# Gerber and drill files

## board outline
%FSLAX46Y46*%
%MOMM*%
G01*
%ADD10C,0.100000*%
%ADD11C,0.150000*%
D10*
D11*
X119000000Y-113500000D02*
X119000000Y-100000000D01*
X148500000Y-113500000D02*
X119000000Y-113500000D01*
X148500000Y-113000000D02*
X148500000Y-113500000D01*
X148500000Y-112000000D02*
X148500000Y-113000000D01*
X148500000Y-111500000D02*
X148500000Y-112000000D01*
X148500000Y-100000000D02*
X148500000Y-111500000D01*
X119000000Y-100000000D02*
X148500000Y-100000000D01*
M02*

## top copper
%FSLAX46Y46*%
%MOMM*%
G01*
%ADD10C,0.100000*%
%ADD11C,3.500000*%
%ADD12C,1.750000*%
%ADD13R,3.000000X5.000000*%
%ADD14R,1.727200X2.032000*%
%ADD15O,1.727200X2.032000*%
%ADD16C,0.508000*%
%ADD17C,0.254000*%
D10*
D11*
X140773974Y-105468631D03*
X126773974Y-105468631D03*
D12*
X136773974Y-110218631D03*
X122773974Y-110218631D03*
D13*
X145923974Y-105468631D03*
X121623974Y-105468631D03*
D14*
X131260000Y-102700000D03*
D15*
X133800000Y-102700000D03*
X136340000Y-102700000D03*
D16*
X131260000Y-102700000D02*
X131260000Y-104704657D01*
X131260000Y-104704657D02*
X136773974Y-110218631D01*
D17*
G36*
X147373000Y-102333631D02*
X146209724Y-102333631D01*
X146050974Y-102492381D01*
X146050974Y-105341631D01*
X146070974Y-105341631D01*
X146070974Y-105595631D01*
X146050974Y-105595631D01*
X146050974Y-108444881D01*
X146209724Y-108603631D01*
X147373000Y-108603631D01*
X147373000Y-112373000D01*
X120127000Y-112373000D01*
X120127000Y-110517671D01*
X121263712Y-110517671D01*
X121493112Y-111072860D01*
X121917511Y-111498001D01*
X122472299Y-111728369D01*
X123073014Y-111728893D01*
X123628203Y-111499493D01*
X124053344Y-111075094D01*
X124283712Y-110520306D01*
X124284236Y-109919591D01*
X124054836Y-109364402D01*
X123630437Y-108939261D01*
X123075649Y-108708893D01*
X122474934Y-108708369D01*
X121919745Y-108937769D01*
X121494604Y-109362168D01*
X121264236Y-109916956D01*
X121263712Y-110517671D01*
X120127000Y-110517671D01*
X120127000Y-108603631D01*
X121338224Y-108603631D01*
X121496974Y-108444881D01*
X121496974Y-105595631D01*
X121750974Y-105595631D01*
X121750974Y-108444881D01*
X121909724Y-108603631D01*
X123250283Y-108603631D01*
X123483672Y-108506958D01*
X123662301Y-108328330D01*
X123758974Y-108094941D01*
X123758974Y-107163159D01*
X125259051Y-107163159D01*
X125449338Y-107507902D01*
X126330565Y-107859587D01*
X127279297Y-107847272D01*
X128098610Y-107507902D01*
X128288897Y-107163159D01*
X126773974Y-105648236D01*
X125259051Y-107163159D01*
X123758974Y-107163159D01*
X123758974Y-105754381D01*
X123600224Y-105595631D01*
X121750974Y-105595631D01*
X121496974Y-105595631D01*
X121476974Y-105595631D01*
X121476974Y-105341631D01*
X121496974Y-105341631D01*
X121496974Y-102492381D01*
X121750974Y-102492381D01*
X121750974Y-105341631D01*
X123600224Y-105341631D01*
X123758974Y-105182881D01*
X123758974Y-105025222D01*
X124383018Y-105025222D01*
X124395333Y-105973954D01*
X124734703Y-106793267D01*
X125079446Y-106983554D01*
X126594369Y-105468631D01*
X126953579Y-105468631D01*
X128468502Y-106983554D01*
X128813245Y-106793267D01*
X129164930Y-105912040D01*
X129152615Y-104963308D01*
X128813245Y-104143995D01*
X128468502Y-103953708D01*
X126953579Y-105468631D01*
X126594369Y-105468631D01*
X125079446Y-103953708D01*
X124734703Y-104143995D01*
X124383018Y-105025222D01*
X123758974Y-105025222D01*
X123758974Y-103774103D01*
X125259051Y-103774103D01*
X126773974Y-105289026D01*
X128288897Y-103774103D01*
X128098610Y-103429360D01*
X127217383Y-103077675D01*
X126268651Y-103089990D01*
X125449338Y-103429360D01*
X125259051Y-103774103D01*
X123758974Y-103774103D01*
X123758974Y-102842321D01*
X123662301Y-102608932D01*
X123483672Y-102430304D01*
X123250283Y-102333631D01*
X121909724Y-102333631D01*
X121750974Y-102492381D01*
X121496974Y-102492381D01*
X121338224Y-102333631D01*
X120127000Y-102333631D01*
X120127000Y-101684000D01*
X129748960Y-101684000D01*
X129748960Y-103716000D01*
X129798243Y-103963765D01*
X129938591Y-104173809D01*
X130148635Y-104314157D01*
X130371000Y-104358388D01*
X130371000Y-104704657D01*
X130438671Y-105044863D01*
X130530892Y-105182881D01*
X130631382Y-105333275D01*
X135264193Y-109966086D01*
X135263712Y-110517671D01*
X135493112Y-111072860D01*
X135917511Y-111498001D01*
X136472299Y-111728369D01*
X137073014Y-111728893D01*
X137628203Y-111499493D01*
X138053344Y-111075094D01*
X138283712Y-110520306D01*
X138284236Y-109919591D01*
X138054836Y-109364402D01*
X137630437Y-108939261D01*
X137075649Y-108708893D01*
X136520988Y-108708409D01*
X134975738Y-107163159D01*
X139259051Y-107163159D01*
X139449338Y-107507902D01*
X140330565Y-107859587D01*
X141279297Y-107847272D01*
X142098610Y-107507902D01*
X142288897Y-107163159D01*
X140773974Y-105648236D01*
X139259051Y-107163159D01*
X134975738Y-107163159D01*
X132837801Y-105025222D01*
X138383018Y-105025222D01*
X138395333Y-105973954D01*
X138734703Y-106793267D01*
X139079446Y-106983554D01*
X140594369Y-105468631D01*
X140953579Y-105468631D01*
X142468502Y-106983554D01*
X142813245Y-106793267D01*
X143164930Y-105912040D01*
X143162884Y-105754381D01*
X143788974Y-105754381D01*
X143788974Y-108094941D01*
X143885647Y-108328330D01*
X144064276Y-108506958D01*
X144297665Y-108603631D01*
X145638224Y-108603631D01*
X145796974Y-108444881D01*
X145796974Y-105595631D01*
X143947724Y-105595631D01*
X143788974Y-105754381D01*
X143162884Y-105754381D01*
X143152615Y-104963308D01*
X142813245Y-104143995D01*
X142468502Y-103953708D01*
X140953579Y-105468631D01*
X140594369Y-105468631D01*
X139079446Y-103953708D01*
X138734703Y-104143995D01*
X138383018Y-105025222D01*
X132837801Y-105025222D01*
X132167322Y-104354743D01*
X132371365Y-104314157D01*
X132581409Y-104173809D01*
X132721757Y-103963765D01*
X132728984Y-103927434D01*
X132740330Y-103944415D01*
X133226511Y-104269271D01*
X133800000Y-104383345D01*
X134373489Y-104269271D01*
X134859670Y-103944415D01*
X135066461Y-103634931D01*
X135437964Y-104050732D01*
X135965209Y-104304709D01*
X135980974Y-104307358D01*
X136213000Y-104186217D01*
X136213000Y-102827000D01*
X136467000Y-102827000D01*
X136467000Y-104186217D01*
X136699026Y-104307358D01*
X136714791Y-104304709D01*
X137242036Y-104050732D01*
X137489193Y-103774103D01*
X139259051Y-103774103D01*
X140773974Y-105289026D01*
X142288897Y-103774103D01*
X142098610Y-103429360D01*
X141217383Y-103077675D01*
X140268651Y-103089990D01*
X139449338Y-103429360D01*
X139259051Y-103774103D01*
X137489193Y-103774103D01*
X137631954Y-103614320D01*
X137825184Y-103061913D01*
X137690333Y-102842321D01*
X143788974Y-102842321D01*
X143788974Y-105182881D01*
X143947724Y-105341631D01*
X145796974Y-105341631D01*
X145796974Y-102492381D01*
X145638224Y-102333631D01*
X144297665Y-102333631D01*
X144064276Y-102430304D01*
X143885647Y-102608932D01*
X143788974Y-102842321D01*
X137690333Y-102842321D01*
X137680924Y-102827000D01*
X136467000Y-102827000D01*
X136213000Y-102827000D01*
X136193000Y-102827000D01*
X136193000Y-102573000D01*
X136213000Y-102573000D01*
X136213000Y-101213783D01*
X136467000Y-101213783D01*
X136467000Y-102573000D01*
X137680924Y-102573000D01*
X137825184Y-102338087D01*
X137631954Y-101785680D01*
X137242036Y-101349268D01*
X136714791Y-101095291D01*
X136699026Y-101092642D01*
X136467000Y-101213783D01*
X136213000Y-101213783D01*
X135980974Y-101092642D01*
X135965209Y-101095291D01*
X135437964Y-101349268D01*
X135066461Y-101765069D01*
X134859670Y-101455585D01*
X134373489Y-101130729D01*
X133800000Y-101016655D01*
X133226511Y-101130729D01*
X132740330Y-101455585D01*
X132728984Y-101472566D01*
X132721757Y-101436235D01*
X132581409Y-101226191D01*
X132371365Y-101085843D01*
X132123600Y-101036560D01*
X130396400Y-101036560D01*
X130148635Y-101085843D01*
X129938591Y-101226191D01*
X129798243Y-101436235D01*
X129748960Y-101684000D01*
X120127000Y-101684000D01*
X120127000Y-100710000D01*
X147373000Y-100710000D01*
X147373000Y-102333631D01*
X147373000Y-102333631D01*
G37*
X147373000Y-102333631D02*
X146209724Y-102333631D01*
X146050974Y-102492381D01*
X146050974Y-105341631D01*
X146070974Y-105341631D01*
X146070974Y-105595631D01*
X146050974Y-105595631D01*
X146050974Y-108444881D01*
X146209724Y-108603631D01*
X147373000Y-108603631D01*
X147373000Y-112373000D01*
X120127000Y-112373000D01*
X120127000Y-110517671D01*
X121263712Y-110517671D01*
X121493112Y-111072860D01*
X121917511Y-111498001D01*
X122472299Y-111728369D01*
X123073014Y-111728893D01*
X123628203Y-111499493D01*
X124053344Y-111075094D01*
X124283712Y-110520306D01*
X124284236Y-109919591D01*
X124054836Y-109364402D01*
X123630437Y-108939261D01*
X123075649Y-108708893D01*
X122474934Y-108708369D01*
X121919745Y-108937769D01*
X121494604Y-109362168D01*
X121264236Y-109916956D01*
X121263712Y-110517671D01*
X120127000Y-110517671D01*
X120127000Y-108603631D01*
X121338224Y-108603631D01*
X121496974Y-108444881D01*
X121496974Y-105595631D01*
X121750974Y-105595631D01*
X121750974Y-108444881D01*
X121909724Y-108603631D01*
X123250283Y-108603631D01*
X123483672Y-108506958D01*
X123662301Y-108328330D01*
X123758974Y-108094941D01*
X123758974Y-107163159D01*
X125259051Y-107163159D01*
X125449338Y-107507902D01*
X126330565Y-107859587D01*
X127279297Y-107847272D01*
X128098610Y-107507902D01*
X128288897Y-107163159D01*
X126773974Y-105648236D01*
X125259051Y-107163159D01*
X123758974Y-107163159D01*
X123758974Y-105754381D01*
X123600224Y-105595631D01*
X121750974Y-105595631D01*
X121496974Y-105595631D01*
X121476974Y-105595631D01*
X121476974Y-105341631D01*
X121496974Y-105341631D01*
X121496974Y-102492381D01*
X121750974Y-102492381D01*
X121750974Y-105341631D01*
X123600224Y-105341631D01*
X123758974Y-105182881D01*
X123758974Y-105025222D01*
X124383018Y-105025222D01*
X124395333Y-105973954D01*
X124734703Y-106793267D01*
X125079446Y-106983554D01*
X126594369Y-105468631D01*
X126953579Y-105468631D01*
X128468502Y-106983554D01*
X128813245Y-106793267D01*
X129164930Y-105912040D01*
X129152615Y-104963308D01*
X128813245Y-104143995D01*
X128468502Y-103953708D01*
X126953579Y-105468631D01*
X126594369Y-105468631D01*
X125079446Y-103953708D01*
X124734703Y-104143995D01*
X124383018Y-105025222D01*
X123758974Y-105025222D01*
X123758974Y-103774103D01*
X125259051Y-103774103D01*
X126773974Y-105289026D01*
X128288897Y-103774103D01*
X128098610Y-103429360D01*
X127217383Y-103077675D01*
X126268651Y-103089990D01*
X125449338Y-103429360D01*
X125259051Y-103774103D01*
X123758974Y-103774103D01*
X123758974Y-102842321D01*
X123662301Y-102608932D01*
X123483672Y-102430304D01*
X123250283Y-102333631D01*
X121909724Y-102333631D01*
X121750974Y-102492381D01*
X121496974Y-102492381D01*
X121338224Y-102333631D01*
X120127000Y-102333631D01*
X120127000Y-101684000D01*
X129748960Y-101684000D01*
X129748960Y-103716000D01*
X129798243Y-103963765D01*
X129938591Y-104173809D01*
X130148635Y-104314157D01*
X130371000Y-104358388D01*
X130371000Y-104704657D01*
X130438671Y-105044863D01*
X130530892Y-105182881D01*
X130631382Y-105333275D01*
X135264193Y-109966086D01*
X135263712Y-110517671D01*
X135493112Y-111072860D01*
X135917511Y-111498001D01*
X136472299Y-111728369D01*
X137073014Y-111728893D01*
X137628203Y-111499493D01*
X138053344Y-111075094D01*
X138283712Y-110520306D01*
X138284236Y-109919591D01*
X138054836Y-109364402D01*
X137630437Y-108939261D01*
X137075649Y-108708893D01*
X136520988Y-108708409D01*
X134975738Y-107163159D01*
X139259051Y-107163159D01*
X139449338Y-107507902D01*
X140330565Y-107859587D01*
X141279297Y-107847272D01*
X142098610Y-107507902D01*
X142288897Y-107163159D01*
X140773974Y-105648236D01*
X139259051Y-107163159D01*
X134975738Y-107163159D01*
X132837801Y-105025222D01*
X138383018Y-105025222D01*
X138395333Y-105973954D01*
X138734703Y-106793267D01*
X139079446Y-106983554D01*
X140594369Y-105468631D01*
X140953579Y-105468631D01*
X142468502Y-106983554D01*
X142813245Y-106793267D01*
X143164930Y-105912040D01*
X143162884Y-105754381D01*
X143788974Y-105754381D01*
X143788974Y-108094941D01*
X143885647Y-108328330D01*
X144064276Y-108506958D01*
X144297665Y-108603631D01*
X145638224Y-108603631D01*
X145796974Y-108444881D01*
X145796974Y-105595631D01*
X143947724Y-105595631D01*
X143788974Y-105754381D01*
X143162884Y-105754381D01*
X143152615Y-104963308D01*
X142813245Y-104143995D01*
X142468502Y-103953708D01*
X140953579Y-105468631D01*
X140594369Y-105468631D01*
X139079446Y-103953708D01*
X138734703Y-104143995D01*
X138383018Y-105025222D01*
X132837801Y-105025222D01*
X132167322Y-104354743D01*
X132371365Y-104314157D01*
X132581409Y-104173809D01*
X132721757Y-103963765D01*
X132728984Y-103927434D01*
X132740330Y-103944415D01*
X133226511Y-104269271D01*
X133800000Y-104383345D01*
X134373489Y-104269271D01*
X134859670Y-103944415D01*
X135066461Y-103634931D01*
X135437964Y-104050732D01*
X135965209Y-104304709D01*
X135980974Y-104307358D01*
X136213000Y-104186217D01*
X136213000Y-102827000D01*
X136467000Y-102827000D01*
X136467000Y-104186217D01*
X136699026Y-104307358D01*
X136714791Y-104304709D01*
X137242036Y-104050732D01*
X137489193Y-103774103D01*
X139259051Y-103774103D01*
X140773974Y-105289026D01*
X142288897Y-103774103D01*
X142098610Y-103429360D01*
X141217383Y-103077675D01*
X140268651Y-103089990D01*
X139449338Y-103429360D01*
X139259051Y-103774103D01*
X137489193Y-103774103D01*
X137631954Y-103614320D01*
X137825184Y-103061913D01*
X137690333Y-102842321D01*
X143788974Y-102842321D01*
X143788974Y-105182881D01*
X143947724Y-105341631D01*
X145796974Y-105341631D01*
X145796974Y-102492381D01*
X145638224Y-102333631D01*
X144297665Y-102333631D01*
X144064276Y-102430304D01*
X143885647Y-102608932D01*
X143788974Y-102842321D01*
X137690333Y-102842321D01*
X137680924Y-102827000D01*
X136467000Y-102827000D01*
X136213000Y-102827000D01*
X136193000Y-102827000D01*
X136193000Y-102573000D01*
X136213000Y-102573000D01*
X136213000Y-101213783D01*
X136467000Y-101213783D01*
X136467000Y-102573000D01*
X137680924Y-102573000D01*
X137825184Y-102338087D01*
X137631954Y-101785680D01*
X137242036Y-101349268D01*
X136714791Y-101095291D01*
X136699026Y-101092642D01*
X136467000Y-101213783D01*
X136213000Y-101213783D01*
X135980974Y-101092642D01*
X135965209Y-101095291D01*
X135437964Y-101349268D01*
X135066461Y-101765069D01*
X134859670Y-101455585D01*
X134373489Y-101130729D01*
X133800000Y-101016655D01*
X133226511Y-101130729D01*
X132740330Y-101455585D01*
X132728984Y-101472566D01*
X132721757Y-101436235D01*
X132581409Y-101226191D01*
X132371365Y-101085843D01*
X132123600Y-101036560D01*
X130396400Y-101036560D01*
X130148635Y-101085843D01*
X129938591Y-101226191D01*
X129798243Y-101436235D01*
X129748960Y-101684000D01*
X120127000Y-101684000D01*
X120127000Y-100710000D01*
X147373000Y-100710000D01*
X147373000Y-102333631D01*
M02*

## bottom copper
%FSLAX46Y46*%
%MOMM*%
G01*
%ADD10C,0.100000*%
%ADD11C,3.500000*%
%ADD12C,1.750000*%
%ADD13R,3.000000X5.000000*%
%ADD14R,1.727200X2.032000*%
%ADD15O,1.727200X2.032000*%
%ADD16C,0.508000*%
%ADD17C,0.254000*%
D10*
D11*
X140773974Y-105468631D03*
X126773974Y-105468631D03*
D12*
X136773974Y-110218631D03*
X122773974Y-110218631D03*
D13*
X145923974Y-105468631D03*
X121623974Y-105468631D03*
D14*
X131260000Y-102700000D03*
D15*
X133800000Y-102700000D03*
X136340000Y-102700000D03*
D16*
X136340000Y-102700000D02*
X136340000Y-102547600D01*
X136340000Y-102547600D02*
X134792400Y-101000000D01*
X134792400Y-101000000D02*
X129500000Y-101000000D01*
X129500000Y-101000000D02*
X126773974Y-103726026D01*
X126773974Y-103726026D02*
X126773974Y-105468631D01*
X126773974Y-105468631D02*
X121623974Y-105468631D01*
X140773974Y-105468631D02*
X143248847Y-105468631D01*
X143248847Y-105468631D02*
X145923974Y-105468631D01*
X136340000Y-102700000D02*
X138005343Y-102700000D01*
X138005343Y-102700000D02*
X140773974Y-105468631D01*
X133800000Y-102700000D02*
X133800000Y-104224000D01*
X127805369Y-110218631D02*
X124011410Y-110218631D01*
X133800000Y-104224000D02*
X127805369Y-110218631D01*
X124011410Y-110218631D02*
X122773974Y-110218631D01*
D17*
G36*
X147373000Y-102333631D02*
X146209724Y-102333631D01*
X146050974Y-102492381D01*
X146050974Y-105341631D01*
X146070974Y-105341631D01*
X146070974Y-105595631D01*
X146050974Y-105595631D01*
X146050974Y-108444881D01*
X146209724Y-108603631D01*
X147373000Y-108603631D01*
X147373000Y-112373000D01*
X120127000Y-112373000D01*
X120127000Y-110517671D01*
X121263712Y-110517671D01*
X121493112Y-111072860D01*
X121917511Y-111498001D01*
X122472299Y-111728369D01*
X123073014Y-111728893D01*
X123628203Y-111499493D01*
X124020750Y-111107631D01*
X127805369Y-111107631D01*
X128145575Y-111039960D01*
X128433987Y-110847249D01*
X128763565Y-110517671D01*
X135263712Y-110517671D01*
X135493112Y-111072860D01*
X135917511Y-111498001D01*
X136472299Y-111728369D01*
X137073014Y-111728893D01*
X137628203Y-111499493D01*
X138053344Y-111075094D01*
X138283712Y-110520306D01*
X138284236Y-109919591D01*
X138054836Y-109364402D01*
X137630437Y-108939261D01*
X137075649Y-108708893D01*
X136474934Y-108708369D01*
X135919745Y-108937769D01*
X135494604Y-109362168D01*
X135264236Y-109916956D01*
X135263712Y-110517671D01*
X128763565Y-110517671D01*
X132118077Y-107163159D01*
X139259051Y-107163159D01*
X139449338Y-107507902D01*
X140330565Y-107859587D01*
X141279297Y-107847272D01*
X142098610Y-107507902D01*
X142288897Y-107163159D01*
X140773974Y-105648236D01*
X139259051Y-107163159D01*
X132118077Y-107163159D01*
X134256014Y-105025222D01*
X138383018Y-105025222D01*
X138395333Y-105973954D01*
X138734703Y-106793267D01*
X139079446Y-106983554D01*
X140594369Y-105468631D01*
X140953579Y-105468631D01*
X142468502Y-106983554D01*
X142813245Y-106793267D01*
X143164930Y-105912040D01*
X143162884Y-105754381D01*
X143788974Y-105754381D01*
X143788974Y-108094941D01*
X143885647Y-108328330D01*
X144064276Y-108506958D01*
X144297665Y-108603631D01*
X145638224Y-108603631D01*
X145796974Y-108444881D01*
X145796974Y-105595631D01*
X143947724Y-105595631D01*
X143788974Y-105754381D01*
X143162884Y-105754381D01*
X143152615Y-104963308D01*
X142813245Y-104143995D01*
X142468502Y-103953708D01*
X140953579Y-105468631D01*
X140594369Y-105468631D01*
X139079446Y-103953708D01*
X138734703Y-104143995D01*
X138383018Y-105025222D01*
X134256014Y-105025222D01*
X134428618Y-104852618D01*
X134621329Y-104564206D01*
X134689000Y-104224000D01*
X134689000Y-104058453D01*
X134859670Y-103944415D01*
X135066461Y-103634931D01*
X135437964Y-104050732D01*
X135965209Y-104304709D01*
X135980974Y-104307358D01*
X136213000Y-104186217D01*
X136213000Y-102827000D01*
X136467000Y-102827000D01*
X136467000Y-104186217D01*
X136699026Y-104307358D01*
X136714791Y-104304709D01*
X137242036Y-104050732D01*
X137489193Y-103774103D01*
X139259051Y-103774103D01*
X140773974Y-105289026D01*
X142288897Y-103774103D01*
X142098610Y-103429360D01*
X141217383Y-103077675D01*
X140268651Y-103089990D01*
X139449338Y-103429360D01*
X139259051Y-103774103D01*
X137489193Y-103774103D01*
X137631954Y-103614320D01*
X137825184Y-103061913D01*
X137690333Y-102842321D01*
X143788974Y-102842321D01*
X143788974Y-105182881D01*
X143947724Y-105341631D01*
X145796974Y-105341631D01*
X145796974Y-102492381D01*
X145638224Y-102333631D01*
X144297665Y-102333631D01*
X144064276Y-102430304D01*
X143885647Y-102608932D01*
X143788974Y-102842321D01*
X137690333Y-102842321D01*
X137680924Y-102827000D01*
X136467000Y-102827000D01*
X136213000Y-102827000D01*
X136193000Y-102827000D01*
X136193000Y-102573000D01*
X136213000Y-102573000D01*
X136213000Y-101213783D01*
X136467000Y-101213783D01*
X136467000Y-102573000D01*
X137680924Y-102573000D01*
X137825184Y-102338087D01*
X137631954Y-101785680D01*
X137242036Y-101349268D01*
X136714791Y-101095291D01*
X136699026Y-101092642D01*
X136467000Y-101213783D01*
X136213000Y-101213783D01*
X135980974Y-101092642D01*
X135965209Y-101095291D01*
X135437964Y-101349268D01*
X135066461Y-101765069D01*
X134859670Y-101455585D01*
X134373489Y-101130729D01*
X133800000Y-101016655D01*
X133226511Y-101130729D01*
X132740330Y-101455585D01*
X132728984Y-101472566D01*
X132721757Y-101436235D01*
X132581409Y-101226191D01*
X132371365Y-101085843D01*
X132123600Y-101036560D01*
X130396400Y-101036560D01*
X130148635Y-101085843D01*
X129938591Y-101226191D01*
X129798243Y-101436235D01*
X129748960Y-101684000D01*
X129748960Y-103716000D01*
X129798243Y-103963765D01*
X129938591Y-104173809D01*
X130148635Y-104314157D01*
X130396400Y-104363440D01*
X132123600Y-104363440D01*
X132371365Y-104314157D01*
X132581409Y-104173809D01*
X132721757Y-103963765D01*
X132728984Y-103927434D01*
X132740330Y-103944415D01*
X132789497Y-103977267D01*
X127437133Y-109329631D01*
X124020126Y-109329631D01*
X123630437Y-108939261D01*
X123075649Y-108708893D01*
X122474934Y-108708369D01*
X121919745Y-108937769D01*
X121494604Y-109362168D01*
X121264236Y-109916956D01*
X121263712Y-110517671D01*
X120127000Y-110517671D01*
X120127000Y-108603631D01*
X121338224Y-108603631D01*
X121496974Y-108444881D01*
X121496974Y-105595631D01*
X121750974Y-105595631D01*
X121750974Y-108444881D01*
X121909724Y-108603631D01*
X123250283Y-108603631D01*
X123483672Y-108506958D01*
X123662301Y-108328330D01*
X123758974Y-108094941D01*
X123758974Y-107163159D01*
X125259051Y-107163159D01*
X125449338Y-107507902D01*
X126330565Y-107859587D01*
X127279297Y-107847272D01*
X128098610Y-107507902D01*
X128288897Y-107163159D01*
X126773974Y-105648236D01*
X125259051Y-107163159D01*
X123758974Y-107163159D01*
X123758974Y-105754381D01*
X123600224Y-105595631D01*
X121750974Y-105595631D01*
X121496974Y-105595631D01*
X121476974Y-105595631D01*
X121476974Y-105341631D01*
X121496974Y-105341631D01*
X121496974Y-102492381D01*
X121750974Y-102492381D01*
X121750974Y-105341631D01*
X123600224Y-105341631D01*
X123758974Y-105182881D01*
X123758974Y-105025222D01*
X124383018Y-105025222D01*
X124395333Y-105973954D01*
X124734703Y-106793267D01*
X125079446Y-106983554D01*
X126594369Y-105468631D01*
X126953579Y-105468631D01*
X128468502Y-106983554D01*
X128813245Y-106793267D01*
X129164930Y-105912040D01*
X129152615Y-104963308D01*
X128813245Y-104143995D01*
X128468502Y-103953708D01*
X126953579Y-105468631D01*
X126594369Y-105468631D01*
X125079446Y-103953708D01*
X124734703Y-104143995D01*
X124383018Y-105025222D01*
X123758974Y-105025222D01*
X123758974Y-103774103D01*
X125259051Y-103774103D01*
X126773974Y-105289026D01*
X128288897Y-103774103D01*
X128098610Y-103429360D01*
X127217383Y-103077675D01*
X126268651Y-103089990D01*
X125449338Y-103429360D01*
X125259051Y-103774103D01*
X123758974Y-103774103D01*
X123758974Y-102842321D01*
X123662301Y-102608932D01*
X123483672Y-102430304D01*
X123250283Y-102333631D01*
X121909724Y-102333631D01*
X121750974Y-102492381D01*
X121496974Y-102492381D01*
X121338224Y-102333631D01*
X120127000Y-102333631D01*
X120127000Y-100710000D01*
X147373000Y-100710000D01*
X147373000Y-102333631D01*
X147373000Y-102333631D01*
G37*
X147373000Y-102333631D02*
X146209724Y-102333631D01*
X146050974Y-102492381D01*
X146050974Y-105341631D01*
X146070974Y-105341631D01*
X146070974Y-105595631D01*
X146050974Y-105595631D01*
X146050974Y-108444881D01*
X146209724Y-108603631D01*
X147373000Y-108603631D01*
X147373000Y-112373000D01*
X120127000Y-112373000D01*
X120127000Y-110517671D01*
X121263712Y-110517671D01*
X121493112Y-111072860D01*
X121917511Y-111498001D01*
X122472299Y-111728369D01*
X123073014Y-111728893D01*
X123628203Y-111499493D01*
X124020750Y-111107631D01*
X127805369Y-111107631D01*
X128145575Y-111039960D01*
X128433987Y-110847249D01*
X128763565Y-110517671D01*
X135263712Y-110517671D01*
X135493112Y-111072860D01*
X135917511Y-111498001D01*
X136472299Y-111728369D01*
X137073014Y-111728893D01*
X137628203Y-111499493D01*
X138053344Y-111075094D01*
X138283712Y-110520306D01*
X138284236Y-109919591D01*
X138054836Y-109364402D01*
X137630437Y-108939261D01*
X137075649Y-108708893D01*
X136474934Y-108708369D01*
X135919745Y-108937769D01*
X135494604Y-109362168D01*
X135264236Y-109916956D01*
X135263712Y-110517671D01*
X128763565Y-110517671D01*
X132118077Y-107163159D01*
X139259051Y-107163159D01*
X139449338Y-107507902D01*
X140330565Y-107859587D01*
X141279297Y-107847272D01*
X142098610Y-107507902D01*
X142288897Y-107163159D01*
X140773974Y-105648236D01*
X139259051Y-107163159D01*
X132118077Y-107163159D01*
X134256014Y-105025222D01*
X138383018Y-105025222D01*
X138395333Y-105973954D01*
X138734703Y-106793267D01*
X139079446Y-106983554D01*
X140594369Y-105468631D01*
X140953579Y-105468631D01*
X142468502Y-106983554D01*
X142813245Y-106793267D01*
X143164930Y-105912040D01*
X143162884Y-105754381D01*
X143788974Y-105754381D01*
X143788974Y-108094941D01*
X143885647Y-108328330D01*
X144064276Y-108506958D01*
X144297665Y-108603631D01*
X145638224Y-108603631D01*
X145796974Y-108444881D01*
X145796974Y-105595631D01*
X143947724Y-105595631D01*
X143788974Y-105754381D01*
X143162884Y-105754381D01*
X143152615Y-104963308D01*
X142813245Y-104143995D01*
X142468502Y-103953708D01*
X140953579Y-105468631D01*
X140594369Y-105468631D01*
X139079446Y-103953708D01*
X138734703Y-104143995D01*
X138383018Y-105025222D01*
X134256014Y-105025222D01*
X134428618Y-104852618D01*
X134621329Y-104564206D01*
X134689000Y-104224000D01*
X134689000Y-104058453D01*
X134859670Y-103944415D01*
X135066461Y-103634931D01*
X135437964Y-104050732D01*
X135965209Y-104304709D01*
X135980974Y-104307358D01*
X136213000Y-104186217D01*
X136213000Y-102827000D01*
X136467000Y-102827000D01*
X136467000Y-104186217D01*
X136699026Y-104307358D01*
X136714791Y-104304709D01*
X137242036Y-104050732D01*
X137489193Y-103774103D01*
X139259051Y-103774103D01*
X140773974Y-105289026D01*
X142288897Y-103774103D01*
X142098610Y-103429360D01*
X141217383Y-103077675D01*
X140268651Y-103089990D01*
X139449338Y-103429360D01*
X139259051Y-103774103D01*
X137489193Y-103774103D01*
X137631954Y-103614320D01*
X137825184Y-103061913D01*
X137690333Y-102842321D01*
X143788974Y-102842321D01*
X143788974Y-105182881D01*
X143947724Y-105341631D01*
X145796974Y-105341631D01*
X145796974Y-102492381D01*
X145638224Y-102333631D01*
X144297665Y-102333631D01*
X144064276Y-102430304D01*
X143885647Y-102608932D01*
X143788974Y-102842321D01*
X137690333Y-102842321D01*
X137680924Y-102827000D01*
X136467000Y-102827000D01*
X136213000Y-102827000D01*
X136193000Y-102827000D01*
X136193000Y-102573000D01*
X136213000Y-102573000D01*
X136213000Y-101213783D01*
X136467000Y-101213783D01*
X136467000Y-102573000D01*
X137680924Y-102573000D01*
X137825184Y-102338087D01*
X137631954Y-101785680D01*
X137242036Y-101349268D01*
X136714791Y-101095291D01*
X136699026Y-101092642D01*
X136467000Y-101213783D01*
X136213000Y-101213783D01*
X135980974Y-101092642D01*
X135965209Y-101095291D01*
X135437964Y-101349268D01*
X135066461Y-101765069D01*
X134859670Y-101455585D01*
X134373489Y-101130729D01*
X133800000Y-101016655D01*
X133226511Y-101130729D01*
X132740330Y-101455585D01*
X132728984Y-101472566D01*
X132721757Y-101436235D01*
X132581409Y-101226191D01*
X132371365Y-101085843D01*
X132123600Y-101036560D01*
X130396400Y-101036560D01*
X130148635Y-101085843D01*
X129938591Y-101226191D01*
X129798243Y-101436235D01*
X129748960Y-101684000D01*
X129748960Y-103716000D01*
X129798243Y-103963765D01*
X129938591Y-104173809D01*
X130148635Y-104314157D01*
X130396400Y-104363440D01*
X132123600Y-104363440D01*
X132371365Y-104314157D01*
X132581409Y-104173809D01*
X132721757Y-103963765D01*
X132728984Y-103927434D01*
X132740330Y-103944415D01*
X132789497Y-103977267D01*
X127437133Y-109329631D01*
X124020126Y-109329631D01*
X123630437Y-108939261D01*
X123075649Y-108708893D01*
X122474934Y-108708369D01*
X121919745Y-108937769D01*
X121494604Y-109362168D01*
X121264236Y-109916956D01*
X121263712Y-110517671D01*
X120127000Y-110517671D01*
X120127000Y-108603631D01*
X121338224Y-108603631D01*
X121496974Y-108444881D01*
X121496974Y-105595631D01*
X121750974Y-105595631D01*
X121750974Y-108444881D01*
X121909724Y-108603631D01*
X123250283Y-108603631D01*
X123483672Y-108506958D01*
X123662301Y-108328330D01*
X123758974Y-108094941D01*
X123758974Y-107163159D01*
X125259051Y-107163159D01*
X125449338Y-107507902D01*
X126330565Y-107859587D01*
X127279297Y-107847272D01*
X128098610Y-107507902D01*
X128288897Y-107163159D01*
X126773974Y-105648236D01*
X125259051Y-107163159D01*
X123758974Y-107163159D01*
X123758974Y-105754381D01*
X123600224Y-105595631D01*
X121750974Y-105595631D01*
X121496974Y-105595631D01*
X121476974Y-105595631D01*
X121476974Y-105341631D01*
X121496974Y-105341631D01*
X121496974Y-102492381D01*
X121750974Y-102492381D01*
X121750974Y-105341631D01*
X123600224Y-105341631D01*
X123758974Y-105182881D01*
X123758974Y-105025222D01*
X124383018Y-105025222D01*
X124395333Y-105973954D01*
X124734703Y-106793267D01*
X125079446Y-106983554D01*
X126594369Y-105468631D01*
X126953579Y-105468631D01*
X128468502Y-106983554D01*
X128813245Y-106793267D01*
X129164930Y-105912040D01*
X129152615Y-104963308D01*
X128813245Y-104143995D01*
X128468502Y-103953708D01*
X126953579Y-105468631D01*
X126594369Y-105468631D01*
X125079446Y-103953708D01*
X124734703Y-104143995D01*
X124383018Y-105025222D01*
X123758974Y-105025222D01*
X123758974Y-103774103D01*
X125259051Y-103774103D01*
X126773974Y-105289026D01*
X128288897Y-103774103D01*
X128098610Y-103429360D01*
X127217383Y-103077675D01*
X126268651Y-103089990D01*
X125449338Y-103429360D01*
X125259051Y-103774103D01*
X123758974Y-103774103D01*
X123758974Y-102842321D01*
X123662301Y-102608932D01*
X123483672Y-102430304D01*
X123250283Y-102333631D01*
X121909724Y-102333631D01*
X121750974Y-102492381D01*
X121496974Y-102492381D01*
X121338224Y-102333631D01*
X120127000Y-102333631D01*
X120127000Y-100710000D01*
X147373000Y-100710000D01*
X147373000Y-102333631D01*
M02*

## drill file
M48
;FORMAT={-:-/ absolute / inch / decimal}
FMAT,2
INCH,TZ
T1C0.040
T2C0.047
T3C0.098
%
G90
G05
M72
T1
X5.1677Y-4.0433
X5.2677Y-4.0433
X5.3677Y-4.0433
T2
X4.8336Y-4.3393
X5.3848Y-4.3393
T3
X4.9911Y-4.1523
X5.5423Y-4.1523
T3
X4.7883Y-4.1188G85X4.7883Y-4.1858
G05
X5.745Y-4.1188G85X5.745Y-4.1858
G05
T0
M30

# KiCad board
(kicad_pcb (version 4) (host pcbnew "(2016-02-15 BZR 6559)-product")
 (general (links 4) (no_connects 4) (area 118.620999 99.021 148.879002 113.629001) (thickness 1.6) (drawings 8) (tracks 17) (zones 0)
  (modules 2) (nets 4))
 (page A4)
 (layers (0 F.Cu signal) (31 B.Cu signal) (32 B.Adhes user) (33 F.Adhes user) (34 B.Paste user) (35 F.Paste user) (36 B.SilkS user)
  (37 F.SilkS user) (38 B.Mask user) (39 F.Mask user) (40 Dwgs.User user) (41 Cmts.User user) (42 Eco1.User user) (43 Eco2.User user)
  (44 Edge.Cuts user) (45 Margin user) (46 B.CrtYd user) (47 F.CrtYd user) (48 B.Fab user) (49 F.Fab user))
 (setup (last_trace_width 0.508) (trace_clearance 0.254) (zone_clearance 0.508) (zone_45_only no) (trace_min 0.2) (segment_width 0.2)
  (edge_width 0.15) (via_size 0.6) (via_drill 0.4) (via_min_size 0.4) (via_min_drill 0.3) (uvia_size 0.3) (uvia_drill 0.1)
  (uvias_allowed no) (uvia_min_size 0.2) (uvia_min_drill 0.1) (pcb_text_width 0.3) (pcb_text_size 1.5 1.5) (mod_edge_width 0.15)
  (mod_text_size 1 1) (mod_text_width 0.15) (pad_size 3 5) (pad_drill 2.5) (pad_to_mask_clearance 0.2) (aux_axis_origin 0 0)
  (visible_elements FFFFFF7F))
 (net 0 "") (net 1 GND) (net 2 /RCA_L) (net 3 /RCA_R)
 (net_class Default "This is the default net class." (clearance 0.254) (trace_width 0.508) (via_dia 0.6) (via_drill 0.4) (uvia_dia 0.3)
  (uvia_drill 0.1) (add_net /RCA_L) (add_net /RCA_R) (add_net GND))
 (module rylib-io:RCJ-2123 (layer F.Cu) (at 133.773974 99.968631)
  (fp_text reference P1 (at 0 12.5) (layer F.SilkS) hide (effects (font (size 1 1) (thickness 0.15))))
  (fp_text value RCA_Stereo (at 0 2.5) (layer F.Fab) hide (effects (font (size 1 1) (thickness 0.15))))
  (pad 1 thru_hole circle (at 7 5.5) (size 3.5 3.5) (drill 2.5) (layers *.Cu *.Mask F.SilkS) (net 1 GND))
  (pad 3 thru_hole circle (at -7 5.5) (size 3.5 3.5) (drill 2.5) (layers *.Cu *.Mask F.SilkS) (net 1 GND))
  (pad 2 thru_hole circle (at 3 10.25) (size 1.75 1.75) (drill 1.2) (layers *.Cu *.Mask F.SilkS) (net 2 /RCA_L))
  (pad 4 thru_hole circle (at -11 10.25) (size 1.75 1.75) (drill 1.2) (layers *.Cu *.Mask F.SilkS) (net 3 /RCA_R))
  (pad "" thru_hole rect (at 12.15 5.5) (size 3 5) (drill oval 2.5 4.2) (layers *.Cu *.Mask F.SilkS) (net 1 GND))
  (pad "" thru_hole rect (at -12.15 5.5) (size 3 5) (drill oval 2.5 4.2) (layers *.Cu *.Mask F.SilkS) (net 1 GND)))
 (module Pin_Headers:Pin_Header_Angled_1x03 (layer B.Cu) (at 131.26 102.7 270)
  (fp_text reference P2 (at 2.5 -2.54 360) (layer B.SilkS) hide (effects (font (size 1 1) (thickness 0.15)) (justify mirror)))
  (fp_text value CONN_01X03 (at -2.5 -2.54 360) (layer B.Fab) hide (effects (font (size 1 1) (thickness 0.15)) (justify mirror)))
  (pad 1 thru_hole rect (at 0 0 270) (size 2.032 1.7272) (drill 1.016) (layers *.Cu *.Mask B.SilkS) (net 2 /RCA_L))
  (pad 2 thru_hole oval (at 0 -2.54 270) (size 2.032 1.7272) (drill 1.016) (layers *.Cu *.Mask B.SilkS) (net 3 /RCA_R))
  (pad 3 thru_hole oval (at 0 -5.08 270) (size 2.032 1.7272) (drill 1.016) (layers *.Cu *.Mask B.SilkS) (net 1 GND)))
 (gr_line (start 119 113.5) (end 119 100) (layer Edge.Cuts) (width 0.15))
 (gr_line (start 148.5 113.5) (end 119 113.5) (layer Edge.Cuts) (width 0.15))
 (gr_line (start 148.5 113) (end 148.5 113.5) (layer Edge.Cuts) (width 0.15))
 (gr_line (start 148.5 112) (end 148.5 113) (layer Edge.Cuts) (width 0.15))
 (gr_line (start 148.5 111.5) (end 148.5 112) (layer Edge.Cuts) (width 0.15))
 (gr_line (start 148.5 100) (end 148.5 111.5) (layer Edge.Cuts) (width 0.15))
 (gr_line (start 119 100) (end 148.5 100) (layer Edge.Cuts) (width 0.15))
 (segment (start 119 100) (end 148.5 100) (width 0.25) (layer Dwgs.User) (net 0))
 (segment (start 136.34 102.7) (end 136.34 102.5476) (width 0.508) (layer B.Cu) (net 1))
 (segment (start 136.34 102.5476) (end 134.7924 101) (width 0.508) (layer B.Cu) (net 1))
 (segment (start 134.7924 101) (end 129.5 101) (width 0.508) (layer B.Cu) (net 1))
 (segment (start 129.5 101) (end 126.773974 103.726026) (width 0.508) (layer B.Cu) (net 1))
 (segment (start 126.773974 103.726026) (end 126.773974 105.468631) (width 0.508) (layer B.Cu) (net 1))
 (segment (start 126.773974 105.468631) (end 121.623974 105.468631) (width 0.508) (layer B.Cu) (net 1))
 (segment (start 140.773974 105.468631) (end 143.248847 105.468631) (width 0.508) (layer B.Cu) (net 1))
 (segment (start 143.248847 105.468631) (end 145.923974 105.468631) (width 0.508) (layer B.Cu) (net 1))
 (segment (start 136.34 102.7) (end 138.005343 102.7) (width 0.508) (layer B.Cu) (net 1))
 (segment (start 138.005343 102.7) (end 140.773974 105.468631) (width 0.508) (layer B.Cu) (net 1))
 (segment (start 131.26 102.7) (end 131.26 104.704657) (width 0.508) (layer F.Cu) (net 2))
 (segment (start 131.26 104.704657) (end 136.773974 110.218631) (width 0.508) (layer F.Cu) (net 2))
 (segment (start 133.8 102.7) (end 133.8 104.224) (width 0.508) (layer B.Cu) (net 3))
 (segment (start 127.805369 110.218631) (end 124.01141 110.218631) (width 0.508) (layer B.Cu) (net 3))
 (segment (start 133.8 104.224) (end 127.805369 110.218631) (width 0.508) (layer B.Cu) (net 3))
 (segment (start 124.01141 110.218631) (end 122.773974 110.218631) (width 0.508) (layer B.Cu) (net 3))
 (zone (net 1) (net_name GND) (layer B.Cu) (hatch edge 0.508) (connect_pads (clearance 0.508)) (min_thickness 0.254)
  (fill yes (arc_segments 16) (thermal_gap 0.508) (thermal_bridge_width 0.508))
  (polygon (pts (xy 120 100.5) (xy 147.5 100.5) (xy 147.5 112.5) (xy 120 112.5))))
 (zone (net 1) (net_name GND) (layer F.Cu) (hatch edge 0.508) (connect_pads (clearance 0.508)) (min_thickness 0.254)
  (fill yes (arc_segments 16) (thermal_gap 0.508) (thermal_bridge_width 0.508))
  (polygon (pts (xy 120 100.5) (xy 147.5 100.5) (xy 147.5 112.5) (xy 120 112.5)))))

